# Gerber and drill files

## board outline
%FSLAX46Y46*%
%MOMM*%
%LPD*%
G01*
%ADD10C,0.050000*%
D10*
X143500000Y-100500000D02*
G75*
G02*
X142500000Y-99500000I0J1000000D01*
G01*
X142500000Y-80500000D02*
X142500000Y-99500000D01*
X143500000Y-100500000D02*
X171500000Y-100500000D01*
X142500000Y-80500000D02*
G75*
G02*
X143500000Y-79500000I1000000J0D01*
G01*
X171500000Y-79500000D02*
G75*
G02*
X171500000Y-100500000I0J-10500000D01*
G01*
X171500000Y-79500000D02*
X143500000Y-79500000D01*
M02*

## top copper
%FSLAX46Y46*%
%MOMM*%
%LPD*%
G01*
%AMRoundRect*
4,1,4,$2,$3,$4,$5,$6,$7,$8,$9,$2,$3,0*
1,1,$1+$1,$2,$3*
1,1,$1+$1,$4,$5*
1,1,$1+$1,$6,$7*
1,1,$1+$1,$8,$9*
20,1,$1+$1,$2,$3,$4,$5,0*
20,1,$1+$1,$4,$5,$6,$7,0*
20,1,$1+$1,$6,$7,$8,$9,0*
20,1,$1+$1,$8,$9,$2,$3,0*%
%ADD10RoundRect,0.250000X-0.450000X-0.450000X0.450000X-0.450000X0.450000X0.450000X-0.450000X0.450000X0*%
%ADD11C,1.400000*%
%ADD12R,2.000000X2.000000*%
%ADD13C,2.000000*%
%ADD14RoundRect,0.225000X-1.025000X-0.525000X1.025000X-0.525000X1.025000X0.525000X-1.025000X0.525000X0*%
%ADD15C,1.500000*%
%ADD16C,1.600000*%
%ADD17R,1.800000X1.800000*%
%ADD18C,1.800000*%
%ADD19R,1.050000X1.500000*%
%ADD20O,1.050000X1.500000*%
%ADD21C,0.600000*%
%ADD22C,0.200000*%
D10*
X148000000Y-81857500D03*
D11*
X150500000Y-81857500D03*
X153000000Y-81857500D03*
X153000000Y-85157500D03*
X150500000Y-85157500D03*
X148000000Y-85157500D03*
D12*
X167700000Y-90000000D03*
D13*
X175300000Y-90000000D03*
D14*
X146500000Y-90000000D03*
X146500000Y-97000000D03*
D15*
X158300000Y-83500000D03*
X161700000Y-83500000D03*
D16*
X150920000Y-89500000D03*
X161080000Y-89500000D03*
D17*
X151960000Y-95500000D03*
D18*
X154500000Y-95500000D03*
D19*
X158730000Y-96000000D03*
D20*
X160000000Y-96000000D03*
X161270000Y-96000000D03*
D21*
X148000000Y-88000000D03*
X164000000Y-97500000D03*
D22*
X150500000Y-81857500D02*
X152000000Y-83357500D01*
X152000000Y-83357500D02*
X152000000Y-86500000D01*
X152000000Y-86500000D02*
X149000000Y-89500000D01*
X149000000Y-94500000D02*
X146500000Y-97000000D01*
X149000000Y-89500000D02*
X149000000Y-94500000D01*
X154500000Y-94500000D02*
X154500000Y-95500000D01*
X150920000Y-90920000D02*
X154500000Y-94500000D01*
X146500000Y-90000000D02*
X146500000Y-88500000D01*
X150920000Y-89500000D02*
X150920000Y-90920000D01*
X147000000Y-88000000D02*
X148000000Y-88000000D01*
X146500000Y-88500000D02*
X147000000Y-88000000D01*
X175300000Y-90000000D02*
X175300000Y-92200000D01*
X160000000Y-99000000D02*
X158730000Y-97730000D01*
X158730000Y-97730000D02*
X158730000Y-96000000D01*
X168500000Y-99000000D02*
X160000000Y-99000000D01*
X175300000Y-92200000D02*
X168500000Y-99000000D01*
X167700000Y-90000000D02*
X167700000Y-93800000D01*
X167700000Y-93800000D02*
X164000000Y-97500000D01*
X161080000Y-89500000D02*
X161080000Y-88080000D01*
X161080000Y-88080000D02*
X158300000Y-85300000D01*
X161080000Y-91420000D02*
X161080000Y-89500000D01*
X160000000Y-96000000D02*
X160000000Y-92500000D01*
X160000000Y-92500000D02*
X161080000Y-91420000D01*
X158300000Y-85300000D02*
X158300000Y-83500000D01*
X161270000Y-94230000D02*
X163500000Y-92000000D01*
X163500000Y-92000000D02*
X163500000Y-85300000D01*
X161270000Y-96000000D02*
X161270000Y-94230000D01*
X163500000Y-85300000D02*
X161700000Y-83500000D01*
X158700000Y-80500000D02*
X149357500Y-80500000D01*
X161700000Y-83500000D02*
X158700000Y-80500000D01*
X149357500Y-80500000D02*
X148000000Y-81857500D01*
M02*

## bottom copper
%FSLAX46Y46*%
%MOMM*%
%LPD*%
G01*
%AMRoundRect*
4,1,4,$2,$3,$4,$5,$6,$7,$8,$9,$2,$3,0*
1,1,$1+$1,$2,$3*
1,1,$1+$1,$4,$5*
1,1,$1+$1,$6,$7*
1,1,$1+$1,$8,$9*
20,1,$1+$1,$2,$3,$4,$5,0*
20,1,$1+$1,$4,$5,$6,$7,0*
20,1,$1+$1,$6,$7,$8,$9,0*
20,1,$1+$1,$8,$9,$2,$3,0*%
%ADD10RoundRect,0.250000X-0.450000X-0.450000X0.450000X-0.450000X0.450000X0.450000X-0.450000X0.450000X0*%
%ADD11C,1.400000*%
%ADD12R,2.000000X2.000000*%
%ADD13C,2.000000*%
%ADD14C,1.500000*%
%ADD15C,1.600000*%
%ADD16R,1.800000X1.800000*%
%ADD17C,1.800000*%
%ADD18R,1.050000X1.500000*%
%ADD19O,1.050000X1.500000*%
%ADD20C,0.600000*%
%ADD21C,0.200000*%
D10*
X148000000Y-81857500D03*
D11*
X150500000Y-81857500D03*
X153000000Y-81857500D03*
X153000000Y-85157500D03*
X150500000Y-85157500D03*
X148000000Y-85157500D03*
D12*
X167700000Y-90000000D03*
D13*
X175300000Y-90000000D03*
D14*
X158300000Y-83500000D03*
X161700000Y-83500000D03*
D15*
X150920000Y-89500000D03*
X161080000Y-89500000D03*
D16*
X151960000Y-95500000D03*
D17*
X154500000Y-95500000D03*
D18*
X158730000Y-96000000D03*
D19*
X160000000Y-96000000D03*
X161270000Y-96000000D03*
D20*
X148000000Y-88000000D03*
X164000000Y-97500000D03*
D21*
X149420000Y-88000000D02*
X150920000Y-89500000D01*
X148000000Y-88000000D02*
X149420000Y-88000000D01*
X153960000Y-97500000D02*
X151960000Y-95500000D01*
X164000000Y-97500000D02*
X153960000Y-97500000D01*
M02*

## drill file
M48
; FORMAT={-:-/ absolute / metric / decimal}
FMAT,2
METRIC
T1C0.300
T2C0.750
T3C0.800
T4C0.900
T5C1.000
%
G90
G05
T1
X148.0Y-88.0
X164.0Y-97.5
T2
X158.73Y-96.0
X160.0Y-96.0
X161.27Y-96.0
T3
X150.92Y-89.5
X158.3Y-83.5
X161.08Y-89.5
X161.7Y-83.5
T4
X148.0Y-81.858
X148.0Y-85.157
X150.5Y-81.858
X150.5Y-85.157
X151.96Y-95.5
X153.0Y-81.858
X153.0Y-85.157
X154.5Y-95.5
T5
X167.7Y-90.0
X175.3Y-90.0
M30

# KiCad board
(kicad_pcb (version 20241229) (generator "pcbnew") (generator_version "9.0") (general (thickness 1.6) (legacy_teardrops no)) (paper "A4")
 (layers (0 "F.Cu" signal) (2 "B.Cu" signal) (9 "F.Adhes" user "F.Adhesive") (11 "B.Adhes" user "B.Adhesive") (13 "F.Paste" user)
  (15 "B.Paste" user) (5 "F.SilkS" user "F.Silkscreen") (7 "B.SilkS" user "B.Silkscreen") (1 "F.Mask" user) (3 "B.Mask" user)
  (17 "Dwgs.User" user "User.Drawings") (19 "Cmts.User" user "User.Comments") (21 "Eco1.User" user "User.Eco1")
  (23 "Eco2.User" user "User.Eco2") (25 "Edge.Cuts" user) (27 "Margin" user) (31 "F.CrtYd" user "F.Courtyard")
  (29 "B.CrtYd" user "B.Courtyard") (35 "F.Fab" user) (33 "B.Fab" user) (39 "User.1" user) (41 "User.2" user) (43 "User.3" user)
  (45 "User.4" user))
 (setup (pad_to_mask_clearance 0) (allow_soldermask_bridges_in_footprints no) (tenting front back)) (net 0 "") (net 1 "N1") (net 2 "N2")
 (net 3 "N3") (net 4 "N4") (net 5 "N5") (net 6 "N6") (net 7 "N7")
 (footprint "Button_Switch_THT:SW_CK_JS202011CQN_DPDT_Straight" (layer "F.Cu") (at 148 81.8575)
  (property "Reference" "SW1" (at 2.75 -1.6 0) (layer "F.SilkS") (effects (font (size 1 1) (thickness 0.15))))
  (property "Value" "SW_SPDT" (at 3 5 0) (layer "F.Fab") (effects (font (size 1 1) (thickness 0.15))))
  (pad "1" thru_hole roundrect (at 0 0) (size 1.4 1.4) (drill 0.9) (layers "*.Cu" "*.Mask") (remove_unused_layers no)
   (roundrect_rratio 0.1785714286) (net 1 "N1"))
  (pad "2" thru_hole circle (at 2.5 0) (size 1.4 1.4) (drill 0.9) (layers "*.Cu" "*.Mask") (remove_unused_layers no) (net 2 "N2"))
  (pad "3" thru_hole circle (at 5 0) (size 1.4 1.4) (drill 0.9) (layers "*.Cu" "*.Mask") (remove_unused_layers no) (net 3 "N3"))
  (pad "4" thru_hole circle (at 5 3.3) (size 1.4 1.4) (drill 0.9) (layers "*.Cu" "*.Mask") (remove_unused_layers no))
  (pad "5" thru_hole circle (at 2.5 3.3) (size 1.4 1.4) (drill 0.9) (layers "*.Cu" "*.Mask") (remove_unused_layers no))
  (pad "6" thru_hole circle (at 0 3.3) (size 1.4 1.4) (drill 0.9) (layers "*.Cu" "*.Mask") (remove_unused_layers no)))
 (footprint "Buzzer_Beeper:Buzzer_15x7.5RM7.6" (layer "F.Cu") (at 167.7 90)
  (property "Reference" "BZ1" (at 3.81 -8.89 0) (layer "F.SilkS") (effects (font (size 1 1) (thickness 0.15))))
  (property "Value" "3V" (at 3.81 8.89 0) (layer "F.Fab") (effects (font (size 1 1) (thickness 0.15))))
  (pad "1" thru_hole rect (at 0 0) (size 2 2) (drill 1) (layers "*.Cu" "*.Mask") (remove_unused_layers no) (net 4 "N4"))
  (pad "2" thru_hole circle (at 7.6 0) (size 2 2) (drill 1) (layers "*.Cu" "*.Mask") (remove_unused_layers no) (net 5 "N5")))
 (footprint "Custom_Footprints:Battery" (layer "F.Cu") (at 146.5 93.5)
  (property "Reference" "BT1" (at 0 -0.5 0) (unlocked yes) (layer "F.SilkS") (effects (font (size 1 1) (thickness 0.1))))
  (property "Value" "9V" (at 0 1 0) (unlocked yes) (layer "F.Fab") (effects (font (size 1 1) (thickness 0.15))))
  (pad "1" smd roundrect (at 0 -3.5) (size 2.5 1.5) (layers "F.Cu" "F.Mask" "F.Paste") (roundrect_rratio 0.15) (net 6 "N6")
   (thermal_bridge_angle 45))
  (pad "2" smd roundrect (at 0 3.5) (size 2.5 1.5) (layers "F.Cu" "F.Mask" "F.Paste") (roundrect_rratio 0.15) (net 2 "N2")
   (thermal_bridge_angle 45)))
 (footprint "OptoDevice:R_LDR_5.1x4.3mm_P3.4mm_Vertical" (layer "F.Cu") (at 158.3 83.5)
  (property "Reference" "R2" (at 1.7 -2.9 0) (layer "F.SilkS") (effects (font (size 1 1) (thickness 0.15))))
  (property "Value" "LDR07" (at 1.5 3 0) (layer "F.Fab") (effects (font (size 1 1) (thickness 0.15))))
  (pad "1" thru_hole circle (at 0 0) (size 1.5 1.5) (drill 0.8) (layers "*.Cu" "*.Mask") (remove_unused_layers no) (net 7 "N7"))
  (pad "2" thru_hole circle (at 3.4 0) (size 1.5 1.5) (drill 0.8) (layers "*.Cu" "*.Mask") (remove_unused_layers no) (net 1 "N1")))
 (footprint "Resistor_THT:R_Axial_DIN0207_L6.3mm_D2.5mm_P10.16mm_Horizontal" (layer "F.Cu") (at 150.92 89.5)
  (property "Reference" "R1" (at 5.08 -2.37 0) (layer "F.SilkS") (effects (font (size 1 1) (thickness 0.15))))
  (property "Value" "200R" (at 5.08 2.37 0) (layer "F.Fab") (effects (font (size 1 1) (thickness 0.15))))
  (pad "1" thru_hole circle (at 0 0) (size 1.6 1.6) (drill 0.8) (layers "*.Cu" "*.Mask") (remove_unused_layers no) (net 6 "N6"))
  (pad "2" thru_hole circle (at 10.16 0) (size 1.6 1.6) (drill 0.8) (layers "*.Cu" "*.Mask") (remove_unused_layers no) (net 7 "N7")))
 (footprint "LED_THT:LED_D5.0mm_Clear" (layer "F.Cu") (at 151.96 95.5)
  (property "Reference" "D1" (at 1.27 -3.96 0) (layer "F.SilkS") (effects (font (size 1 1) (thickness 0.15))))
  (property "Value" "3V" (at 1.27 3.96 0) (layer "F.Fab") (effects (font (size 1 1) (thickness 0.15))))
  (pad "1" thru_hole rect (at 0 0) (size 1.8 1.8) (drill 0.9) (layers "*.Cu" "*.Mask") (remove_unused_layers no) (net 4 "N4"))
  (pad "2" thru_hole circle (at 2.54 0) (size 1.8 1.8) (drill 0.9) (layers "*.Cu" "*.Mask") (remove_unused_layers no) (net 6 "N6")))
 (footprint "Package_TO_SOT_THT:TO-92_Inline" (layer "F.Cu") (at 158.73 96)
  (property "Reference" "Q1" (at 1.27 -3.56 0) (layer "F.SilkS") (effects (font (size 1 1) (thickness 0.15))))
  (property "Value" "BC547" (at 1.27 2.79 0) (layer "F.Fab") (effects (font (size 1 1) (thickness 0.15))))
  (pad "1" thru_hole rect (at 0 0) (size 1.05 1.5) (drill 0.75) (layers "*.Cu" "*.Mask") (remove_unused_layers no) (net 5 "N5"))
  (pad "2" thru_hole oval (at 1.27 0) (size 1.05 1.5) (drill 0.75) (layers "*.Cu" "*.Mask") (remove_unused_layers no) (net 7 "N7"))
  (pad "3" thru_hole oval (at 2.54 0) (size 1.05 1.5) (drill 0.75) (layers "*.Cu" "*.Mask") (remove_unused_layers no) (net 1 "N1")))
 (gr_arc (start 143.5 100.5) (mid 142.792893 100.207107) (end 142.5 99.5) (stroke (width 0.05) (type default)) (layer "Edge.Cuts"))
 (gr_line (start 142.5 80.5) (end 142.5 99.5) (stroke (width 0.05) (type default)) (layer "Edge.Cuts"))
 (gr_line (start 143.5 100.5) (end 171.5 100.5) (stroke (width 0.05) (type default)) (layer "Edge.Cuts"))
 (gr_arc (start 142.5 80.5) (mid 142.792893 79.792893) (end 143.5 79.5) (stroke (width 0.05) (type default)) (layer "Edge.Cuts"))
 (gr_arc (start 171.5 79.5) (mid 182 90) (end 171.5 100.5) (stroke (width 0.05) (type default)) (layer "Edge.Cuts"))
 (gr_line (start 171.5 79.5) (end 143.5 79.5) (stroke (width 0.05) (type default)) (layer "Edge.Cuts"))
 (segment (start 150.5 81.8575) (end 152 83.3575) (width 0.2) (layer "F.Cu") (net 2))
 (segment (start 152 83.3575) (end 152 86.5) (width 0.2) (layer "F.Cu") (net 2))
 (segment (start 152 86.5) (end 149 89.5) (width 0.2) (layer "F.Cu") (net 2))
 (segment (start 149 94.5) (end 146.5 97) (width 0.2) (layer "F.Cu") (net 2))
 (segment (start 149 89.5) (end 149 94.5) (width 0.2) (layer "F.Cu") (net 2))
 (segment (start 154.5 94.5) (end 154.5 95.5) (width 0.2) (layer "F.Cu") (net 6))
 (segment (start 150.92 90.92) (end 154.5 94.5) (width 0.2) (layer "F.Cu") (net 6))
 (segment (start 146.5 90) (end 146.5 88.5) (width 0.2) (layer "F.Cu") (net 6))
 (segment (start 150.92 89.5) (end 150.92 90.92) (width 0.2) (layer "F.Cu") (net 6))
 (segment (start 147 88) (end 148 88) (width 0.2) (layer "F.Cu") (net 6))
 (segment (start 146.5 88.5) (end 147 88) (width 0.2) (layer "F.Cu") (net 6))
 (via (at 148 88) (size 0.6) (drill 0.3) (layers "F.Cu" "B.Cu") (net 6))
 (segment (start 149.42 88) (end 150.92 89.5) (width 0.2) (layer "B.Cu") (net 6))
 (segment (start 148 88) (end 149.42 88) (width 0.2) (layer "B.Cu") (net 6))
 (segment (start 175.3 90) (end 175.3 92.2) (width 0.2) (layer "F.Cu") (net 5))
 (segment (start 160 99) (end 158.73 97.73) (width 0.2) (layer "F.Cu") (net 5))
 (segment (start 158.73 97.73) (end 158.73 96) (width 0.2) (layer "F.Cu") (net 5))
 (segment (start 168.5 99) (end 160 99) (width 0.2) (layer "F.Cu") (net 5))
 (segment (start 175.3 92.2) (end 168.5 99) (width 0.2) (layer "F.Cu") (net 5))
 (segment (start 167.7 90) (end 167.7 93.8) (width 0.2) (layer "F.Cu") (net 4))
 (segment (start 167.7 93.8) (end 164 97.5) (width 0.2) (layer "F.Cu") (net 4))
 (via (at 164 97.5) (size 0.6) (drill 0.3) (layers "F.Cu" "B.Cu") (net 4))
 (segment (start 153.96 97.5) (end 151.96 95.5) (width 0.2) (layer "B.Cu") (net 4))
 (segment (start 164 97.5) (end 153.96 97.5) (width 0.2) (layer "B.Cu") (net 4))
 (segment (start 161.08 89.5) (end 161.08 88.08) (width 0.2) (layer "F.Cu") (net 7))
 (segment (start 161.08 88.08) (end 158.3 85.3) (width 0.2) (layer "F.Cu") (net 7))
 (segment (start 161.08 91.42) (end 161.08 89.5) (width 0.2) (layer "F.Cu") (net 7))
 (segment (start 160 96) (end 160 92.5) (width 0.2) (layer "F.Cu") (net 7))
 (segment (start 160 92.5) (end 161.08 91.42) (width 0.2) (layer "F.Cu") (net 7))
 (segment (start 158.3 85.3) (end 158.3 83.5) (width 0.2) (layer "F.Cu") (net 7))
 (segment (start 161.27 94.23) (end 163.5 92) (width 0.2) (layer "F.Cu") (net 1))
 (segment (start 163.5 92) (end 163.5 85.3) (width 0.2) (layer "F.Cu") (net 1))
 (segment (start 161.27 96) (end 161.27 94.23) (width 0.2) (layer "F.Cu") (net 1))
 (segment (start 163.5 85.3) (end 161.7 83.5) (width 0.2) (layer "F.Cu") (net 1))
 (segment (start 158.7 80.5) (end 149.3575 80.5) (width 0.2) (layer "F.Cu") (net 1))
 (segment (start 161.7 83.5) (end 158.7 80.5) (width 0.2) (layer "F.Cu") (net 1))
 (segment (start 149.3575 80.5) (end 148 81.8575) (width 0.2) (layer "F.Cu") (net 1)))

